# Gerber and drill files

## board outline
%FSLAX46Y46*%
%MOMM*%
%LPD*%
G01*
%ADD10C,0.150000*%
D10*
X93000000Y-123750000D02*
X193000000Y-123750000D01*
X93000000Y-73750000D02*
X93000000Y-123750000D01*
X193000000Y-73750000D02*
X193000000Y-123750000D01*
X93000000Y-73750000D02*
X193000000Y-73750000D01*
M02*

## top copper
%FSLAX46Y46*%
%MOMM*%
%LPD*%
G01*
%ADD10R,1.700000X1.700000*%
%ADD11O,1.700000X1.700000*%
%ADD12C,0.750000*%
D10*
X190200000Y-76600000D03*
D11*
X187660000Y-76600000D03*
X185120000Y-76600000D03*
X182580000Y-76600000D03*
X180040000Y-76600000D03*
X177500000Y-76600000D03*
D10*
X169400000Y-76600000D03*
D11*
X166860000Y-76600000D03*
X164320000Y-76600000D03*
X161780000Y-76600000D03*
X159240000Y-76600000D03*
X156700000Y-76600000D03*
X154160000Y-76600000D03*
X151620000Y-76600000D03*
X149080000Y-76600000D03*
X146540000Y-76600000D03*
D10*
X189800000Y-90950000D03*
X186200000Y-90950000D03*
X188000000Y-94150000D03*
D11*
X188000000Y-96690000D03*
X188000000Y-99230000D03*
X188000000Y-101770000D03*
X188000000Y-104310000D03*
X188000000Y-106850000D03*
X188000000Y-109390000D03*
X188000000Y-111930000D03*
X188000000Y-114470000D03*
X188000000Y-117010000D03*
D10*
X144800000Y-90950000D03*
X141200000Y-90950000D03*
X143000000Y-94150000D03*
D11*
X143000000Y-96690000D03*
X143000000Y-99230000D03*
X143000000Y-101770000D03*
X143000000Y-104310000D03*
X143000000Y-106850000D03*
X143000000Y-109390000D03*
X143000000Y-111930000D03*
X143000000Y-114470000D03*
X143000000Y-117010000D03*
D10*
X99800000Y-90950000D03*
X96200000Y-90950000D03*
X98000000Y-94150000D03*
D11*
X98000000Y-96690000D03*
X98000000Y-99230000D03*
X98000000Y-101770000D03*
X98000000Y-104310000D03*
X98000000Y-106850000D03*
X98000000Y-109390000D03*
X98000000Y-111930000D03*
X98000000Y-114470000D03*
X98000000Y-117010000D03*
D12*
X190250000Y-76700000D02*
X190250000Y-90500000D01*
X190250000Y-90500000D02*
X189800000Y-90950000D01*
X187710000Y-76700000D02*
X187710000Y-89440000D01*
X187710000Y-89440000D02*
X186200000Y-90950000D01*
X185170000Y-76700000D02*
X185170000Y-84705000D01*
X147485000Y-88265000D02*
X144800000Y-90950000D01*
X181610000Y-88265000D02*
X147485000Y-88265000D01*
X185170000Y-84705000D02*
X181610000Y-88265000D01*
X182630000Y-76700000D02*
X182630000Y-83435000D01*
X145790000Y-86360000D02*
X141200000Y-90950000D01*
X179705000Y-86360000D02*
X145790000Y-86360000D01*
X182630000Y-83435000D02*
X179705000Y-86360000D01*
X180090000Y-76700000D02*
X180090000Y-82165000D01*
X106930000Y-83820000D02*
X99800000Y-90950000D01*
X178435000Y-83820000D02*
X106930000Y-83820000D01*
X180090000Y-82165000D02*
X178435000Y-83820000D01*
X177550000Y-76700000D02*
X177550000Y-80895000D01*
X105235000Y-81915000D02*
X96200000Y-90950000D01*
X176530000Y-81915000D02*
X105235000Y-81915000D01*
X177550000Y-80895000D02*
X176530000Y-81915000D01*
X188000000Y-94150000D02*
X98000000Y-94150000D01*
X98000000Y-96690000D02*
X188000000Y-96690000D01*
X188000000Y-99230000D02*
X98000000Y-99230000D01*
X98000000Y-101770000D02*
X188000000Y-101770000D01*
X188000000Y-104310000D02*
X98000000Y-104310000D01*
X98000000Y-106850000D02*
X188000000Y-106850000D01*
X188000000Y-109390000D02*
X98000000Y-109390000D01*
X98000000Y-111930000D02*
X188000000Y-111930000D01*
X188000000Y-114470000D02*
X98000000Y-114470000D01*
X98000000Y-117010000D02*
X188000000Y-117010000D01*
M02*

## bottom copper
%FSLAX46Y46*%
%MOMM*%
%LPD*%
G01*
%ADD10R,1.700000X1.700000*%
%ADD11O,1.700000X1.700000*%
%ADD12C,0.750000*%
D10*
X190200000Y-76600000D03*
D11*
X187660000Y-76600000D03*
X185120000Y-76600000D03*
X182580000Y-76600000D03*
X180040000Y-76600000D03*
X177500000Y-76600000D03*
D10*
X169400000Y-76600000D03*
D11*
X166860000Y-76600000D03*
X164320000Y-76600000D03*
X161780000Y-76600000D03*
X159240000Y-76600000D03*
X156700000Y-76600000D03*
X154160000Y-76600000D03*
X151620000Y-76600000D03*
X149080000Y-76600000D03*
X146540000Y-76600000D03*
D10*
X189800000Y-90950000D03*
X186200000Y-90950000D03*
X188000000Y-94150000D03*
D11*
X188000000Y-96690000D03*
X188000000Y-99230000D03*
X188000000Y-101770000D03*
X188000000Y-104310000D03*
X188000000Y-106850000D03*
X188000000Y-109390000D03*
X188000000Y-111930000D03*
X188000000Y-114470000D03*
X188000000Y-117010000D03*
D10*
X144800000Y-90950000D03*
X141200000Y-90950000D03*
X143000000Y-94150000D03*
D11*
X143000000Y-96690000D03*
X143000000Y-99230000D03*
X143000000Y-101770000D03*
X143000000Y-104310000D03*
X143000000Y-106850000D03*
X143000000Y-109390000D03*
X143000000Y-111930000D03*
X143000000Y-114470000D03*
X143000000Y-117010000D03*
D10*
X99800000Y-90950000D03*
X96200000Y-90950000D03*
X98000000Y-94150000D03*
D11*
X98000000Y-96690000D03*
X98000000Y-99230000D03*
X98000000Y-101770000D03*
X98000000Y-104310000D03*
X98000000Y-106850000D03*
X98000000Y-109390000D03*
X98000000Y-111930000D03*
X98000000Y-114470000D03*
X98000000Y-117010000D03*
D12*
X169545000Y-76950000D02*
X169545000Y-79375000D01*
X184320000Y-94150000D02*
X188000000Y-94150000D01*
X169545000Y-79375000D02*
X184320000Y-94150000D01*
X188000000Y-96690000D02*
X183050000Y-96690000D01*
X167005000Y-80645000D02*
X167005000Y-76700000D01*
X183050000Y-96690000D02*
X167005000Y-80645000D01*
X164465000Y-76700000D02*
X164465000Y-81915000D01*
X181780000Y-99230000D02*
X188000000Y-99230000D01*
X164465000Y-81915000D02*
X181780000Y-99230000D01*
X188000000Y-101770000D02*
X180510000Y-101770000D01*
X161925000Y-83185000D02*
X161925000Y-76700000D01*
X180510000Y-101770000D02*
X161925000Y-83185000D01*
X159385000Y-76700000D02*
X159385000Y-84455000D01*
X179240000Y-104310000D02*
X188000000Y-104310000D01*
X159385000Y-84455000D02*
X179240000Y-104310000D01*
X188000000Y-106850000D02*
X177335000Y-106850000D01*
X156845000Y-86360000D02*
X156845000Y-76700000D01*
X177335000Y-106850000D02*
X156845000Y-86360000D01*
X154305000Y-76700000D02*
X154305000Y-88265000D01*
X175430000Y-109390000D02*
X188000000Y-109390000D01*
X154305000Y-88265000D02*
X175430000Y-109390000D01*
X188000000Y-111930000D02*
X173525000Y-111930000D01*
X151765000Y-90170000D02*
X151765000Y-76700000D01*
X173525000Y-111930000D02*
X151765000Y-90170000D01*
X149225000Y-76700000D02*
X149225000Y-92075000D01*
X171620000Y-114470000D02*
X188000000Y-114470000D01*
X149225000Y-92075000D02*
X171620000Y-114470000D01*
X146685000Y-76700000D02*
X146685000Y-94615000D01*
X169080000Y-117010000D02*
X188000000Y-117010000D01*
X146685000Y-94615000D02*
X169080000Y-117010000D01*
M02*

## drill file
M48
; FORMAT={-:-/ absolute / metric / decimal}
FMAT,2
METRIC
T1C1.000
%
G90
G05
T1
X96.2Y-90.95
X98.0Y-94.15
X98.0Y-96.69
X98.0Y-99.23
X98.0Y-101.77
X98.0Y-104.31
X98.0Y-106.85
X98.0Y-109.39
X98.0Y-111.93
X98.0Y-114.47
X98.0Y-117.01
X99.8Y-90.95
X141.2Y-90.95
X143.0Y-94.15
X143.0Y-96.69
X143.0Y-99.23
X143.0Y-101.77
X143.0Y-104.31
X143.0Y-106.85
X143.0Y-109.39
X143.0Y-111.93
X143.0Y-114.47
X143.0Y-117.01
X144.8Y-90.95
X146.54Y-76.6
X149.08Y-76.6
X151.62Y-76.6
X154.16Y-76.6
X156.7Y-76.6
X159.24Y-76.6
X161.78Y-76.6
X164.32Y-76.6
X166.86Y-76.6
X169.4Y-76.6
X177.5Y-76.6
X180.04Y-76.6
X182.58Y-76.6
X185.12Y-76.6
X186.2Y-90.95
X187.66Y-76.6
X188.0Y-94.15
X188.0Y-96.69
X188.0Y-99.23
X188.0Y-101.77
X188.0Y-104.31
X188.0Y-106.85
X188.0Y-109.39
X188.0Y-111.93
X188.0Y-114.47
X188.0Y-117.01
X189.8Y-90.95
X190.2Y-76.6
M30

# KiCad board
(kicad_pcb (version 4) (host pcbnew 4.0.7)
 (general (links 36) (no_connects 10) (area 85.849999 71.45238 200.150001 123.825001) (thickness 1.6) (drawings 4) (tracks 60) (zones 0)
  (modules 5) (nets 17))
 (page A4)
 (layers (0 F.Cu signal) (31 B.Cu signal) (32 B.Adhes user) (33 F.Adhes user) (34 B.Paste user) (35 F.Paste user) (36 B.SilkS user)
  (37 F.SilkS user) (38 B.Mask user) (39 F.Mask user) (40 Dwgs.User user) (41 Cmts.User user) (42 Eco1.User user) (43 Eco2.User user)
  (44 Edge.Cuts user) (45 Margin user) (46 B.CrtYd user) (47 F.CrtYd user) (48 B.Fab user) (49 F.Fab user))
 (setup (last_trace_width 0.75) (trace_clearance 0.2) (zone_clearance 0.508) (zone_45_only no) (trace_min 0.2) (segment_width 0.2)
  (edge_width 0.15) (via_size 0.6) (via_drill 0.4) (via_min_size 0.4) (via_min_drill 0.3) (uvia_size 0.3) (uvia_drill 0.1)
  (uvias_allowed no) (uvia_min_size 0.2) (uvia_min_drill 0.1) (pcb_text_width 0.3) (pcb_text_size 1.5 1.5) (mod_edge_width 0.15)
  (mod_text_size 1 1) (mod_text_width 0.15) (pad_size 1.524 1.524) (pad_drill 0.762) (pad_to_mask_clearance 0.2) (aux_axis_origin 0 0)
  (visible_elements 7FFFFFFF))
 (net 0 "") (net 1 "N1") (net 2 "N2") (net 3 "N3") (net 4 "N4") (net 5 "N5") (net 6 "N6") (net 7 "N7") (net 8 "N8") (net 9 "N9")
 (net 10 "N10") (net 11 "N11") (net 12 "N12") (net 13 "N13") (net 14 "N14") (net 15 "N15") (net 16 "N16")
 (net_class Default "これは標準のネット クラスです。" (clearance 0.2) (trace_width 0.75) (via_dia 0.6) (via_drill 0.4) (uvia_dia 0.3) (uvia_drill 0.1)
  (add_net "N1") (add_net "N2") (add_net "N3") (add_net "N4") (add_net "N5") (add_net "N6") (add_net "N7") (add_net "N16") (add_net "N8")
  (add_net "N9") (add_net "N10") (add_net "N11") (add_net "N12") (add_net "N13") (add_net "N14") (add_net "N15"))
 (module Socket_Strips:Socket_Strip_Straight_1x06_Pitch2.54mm (layer F.Cu) (at 190.2 76.6 270)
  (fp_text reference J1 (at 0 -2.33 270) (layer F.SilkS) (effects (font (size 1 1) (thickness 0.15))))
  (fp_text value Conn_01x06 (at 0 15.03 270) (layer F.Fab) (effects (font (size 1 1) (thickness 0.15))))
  (pad 1 thru_hole rect (at 0 0 270) (size 1.7 1.7) (drill 1) (layers *.Cu *.Mask) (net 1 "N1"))
  (pad 2 thru_hole oval (at 0 2.54 270) (size 1.7 1.7) (drill 1) (layers *.Cu *.Mask) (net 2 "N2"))
  (pad 3 thru_hole oval (at 0 5.08 270) (size 1.7 1.7) (drill 1) (layers *.Cu *.Mask) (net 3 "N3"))
  (pad 4 thru_hole oval (at 0 7.62 270) (size 1.7 1.7) (drill 1) (layers *.Cu *.Mask) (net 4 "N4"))
  (pad 5 thru_hole oval (at 0 10.16 270) (size 1.7 1.7) (drill 1) (layers *.Cu *.Mask) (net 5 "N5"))
  (pad 6 thru_hole oval (at 0 12.7 270) (size 1.7 1.7) (drill 1) (layers *.Cu *.Mask) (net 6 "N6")))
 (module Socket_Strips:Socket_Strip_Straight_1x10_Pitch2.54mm (layer F.Cu) (at 169.4 76.6 270)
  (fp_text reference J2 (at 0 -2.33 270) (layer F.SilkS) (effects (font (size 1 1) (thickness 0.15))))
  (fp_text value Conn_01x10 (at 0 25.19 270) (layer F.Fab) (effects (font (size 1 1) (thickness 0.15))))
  (pad 1 thru_hole rect (at 0 0 270) (size 1.7 1.7) (drill 1) (layers *.Cu *.Mask) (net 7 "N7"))
  (pad 2 thru_hole oval (at 0 2.54 270) (size 1.7 1.7) (drill 1) (layers *.Cu *.Mask) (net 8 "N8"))
  (pad 3 thru_hole oval (at 0 5.08 270) (size 1.7 1.7) (drill 1) (layers *.Cu *.Mask) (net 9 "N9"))
  (pad 4 thru_hole oval (at 0 7.62 270) (size 1.7 1.7) (drill 1) (layers *.Cu *.Mask) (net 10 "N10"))
  (pad 5 thru_hole oval (at 0 10.16 270) (size 1.7 1.7) (drill 1) (layers *.Cu *.Mask) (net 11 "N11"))
  (pad 6 thru_hole oval (at 0 12.7 270) (size 1.7 1.7) (drill 1) (layers *.Cu *.Mask) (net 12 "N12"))
  (pad 7 thru_hole oval (at 0 15.24 270) (size 1.7 1.7) (drill 1) (layers *.Cu *.Mask) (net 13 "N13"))
  (pad 8 thru_hole oval (at 0 17.78 270) (size 1.7 1.7) (drill 1) (layers *.Cu *.Mask) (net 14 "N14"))
  (pad 9 thru_hole oval (at 0 20.32 270) (size 1.7 1.7) (drill 1) (layers *.Cu *.Mask) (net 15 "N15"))
  (pad 10 thru_hole oval (at 0 22.86 270) (size 1.7 1.7) (drill 1) (layers *.Cu *.Mask) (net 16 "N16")))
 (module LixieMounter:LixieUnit (layer F.Cu) (at 188 94.55)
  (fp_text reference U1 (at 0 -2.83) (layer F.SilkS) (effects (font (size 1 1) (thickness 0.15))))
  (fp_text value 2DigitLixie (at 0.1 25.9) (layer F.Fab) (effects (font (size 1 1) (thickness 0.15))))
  (pad 1 thru_hole rect (at 1.8 -3.6) (size 1.7 1.7) (drill 1) (layers *.Cu *.Mask) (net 1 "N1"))
  (pad 2 thru_hole rect (at -1.8 -3.6) (size 1.7 1.7) (drill 1) (layers *.Cu *.Mask) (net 2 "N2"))
  (pad 3 thru_hole rect (at 0 -0.4) (size 1.7 1.7) (drill 1) (layers *.Cu *.Mask) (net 7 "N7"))
  (pad 4 thru_hole oval (at 0 2.14) (size 1.7 1.7) (drill 1) (layers *.Cu *.Mask) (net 8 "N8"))
  (pad 5 thru_hole oval (at 0 4.68) (size 1.7 1.7) (drill 1) (layers *.Cu *.Mask) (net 9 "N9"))
  (pad 6 thru_hole oval (at 0 7.22) (size 1.7 1.7) (drill 1) (layers *.Cu *.Mask) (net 10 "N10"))
  (pad 7 thru_hole oval (at 0 9.76) (size 1.7 1.7) (drill 1) (layers *.Cu *.Mask) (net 11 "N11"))
  (pad 8 thru_hole oval (at 0 12.3) (size 1.7 1.7) (drill 1) (layers *.Cu *.Mask) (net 12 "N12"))
  (pad 9 thru_hole oval (at 0 14.84) (size 1.7 1.7) (drill 1) (layers *.Cu *.Mask) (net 13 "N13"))
  (pad 10 thru_hole oval (at 0 17.38) (size 1.7 1.7) (drill 1) (layers *.Cu *.Mask) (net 14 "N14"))
  (pad 11 thru_hole oval (at 0 19.92) (size 1.7 1.7) (drill 1) (layers *.Cu *.Mask) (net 15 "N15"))
  (pad 12 thru_hole oval (at 0 22.46) (size 1.7 1.7) (drill 1) (layers *.Cu *.Mask) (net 16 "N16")))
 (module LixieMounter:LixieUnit (layer F.Cu) (at 143 94.55)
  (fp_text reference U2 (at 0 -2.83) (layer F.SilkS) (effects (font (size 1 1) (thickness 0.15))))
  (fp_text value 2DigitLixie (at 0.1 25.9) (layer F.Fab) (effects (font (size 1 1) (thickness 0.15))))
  (pad 1 thru_hole rect (at 1.8 -3.6) (size 1.7 1.7) (drill 1) (layers *.Cu *.Mask) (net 3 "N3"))
  (pad 2 thru_hole rect (at -1.8 -3.6) (size 1.7 1.7) (drill 1) (layers *.Cu *.Mask) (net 4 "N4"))
  (pad 3 thru_hole rect (at 0 -0.4) (size 1.7 1.7) (drill 1) (layers *.Cu *.Mask) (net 7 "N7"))
  (pad 4 thru_hole oval (at 0 2.14) (size 1.7 1.7) (drill 1) (layers *.Cu *.Mask) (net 8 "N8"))
  (pad 5 thru_hole oval (at 0 4.68) (size 1.7 1.7) (drill 1) (layers *.Cu *.Mask) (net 9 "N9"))
  (pad 6 thru_hole oval (at 0 7.22) (size 1.7 1.7) (drill 1) (layers *.Cu *.Mask) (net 10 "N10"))
  (pad 7 thru_hole oval (at 0 9.76) (size 1.7 1.7) (drill 1) (layers *.Cu *.Mask) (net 11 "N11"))
  (pad 8 thru_hole oval (at 0 12.3) (size 1.7 1.7) (drill 1) (layers *.Cu *.Mask) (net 12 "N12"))
  (pad 9 thru_hole oval (at 0 14.84) (size 1.7 1.7) (drill 1) (layers *.Cu *.Mask) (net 13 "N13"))
  (pad 10 thru_hole oval (at 0 17.38) (size 1.7 1.7) (drill 1) (layers *.Cu *.Mask) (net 14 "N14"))
  (pad 11 thru_hole oval (at 0 19.92) (size 1.7 1.7) (drill 1) (layers *.Cu *.Mask) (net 15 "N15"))
  (pad 12 thru_hole oval (at 0 22.46) (size 1.7 1.7) (drill 1) (layers *.Cu *.Mask) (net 16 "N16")))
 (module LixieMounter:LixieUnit (layer F.Cu) (at 98 94.55)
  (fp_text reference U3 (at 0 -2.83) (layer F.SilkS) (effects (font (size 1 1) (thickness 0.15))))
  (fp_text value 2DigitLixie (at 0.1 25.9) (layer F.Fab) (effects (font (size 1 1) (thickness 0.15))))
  (pad 1 thru_hole rect (at 1.8 -3.6) (size 1.7 1.7) (drill 1) (layers *.Cu *.Mask) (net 5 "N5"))
  (pad 2 thru_hole rect (at -1.8 -3.6) (size 1.7 1.7) (drill 1) (layers *.Cu *.Mask) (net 6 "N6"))
  (pad 3 thru_hole rect (at 0 -0.4) (size 1.7 1.7) (drill 1) (layers *.Cu *.Mask) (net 7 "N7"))
  (pad 4 thru_hole oval (at 0 2.14) (size 1.7 1.7) (drill 1) (layers *.Cu *.Mask) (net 8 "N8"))
  (pad 5 thru_hole oval (at 0 4.68) (size 1.7 1.7) (drill 1) (layers *.Cu *.Mask) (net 9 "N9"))
  (pad 6 thru_hole oval (at 0 7.22) (size 1.7 1.7) (drill 1) (layers *.Cu *.Mask) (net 10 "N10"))
  (pad 7 thru_hole oval (at 0 9.76) (size 1.7 1.7) (drill 1) (layers *.Cu *.Mask) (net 11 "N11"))
  (pad 8 thru_hole oval (at 0 12.3) (size 1.7 1.7) (drill 1) (layers *.Cu *.Mask) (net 12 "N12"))
  (pad 9 thru_hole oval (at 0 14.84) (size 1.7 1.7) (drill 1) (layers *.Cu *.Mask) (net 13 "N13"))
  (pad 10 thru_hole oval (at 0 17.38) (size 1.7 1.7) (drill 1) (layers *.Cu *.Mask) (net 14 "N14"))
  (pad 11 thru_hole oval (at 0 19.92) (size 1.7 1.7) (drill 1) (layers *.Cu *.Mask) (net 15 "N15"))
  (pad 12 thru_hole oval (at 0 22.46) (size 1.7 1.7) (drill 1) (layers *.Cu *.Mask) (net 16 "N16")))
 (gr_line (start 93 123.75) (end 193 123.75) (angle 90) (layer Edge.Cuts) (width 0.15))
 (gr_line (start 93 73.75) (end 93 123.75) (angle 90) (layer Edge.Cuts) (width 0.15))
 (gr_line (start 193 73.75) (end 193 123.75) (angle 90) (layer Edge.Cuts) (width 0.15))
 (gr_line (start 93 73.75) (end 193 73.75) (angle 90) (layer Edge.Cuts) (width 0.15))
 (segment (start 190.25 76.7) (end 190.25 90.5) (width 0.75) (layer F.Cu) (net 1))
 (segment (start 190.25 90.5) (end 189.8 90.95) (width 0.75) (layer F.Cu) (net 1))
 (segment (start 187.71 76.7) (end 187.71 89.44) (width 0.75) (layer F.Cu) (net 2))
 (segment (start 187.71 89.44) (end 186.2 90.95) (width 0.75) (layer F.Cu) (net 2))
 (segment (start 185.17 76.7) (end 185.17 84.705) (width 0.75) (layer F.Cu) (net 3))
 (segment (start 147.485 88.265) (end 144.8 90.95) (width 0.75) (layer F.Cu) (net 3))
 (segment (start 181.61 88.265) (end 147.485 88.265) (width 0.75) (layer F.Cu) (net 3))
 (segment (start 185.17 84.705) (end 181.61 88.265) (width 0.75) (layer F.Cu) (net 3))
 (segment (start 182.63 76.7) (end 182.63 83.435) (width 0.75) (layer F.Cu) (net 4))
 (segment (start 145.79 86.36) (end 141.2 90.95) (width 0.75) (layer F.Cu) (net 4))
 (segment (start 179.705 86.36) (end 145.79 86.36) (width 0.75) (layer F.Cu) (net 4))
 (segment (start 182.63 83.435) (end 179.705 86.36) (width 0.75) (layer F.Cu) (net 4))
 (segment (start 180.09 76.7) (end 180.09 82.165) (width 0.75) (layer F.Cu) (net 5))
 (segment (start 106.93 83.82) (end 99.8 90.95) (width 0.75) (layer F.Cu) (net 5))
 (segment (start 178.435 83.82) (end 106.93 83.82) (width 0.75) (layer F.Cu) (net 5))
 (segment (start 180.09 82.165) (end 178.435 83.82) (width 0.75) (layer F.Cu) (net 5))
 (segment (start 177.55 76.7) (end 177.55 80.895) (width 0.75) (layer F.Cu) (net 6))
 (segment (start 105.235 81.915) (end 96.2 90.95) (width 0.75) (layer F.Cu) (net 6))
 (segment (start 176.53 81.915) (end 105.235 81.915) (width 0.75) (layer F.Cu) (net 6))
 (segment (start 177.55 80.895) (end 176.53 81.915) (width 0.75) (layer F.Cu) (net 6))
 (segment (start 169.545 76.95) (end 169.545 79.375) (width 0.75) (layer B.Cu) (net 7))
 (segment (start 184.32 94.15) (end 188 94.15) (width 0.75) (layer B.Cu) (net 7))
 (segment (start 169.545 79.375) (end 184.32 94.15) (width 0.75) (layer B.Cu) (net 7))
 (segment (start 188 94.15) (end 98 94.15) (width 0.75) (layer F.Cu) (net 7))
 (segment (start 188 96.69) (end 183.05 96.69) (width 0.75) (layer B.Cu) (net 8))
 (segment (start 167.005 80.645) (end 167.005 76.7) (width 0.75) (layer B.Cu) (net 8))
 (segment (start 183.05 96.69) (end 167.005 80.645) (width 0.75) (layer B.Cu) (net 8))
 (segment (start 98 96.69) (end 188 96.69) (width 0.75) (layer F.Cu) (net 8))
 (segment (start 164.465 76.7) (end 164.465 81.915) (width 0.75) (layer B.Cu) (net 9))
 (segment (start 181.78 99.23) (end 188 99.23) (width 0.75) (layer B.Cu) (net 9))
 (segment (start 164.465 81.915) (end 181.78 99.23) (width 0.75) (layer B.Cu) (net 9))
 (segment (start 188 99.23) (end 98 99.23) (width 0.75) (layer F.Cu) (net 9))
 (segment (start 188 101.77) (end 180.51 101.77) (width 0.75) (layer B.Cu) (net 10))
 (segment (start 161.925 83.185) (end 161.925 76.7) (width 0.75) (layer B.Cu) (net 10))
 (segment (start 180.51 101.77) (end 161.925 83.185) (width 0.75) (layer B.Cu) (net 10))
 (segment (start 98 101.77) (end 188 101.77) (width 0.75) (layer F.Cu) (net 10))
 (segment (start 159.385 76.7) (end 159.385 84.455) (width 0.75) (layer B.Cu) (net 11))
 (segment (start 179.24 104.31) (end 188 104.31) (width 0.75) (layer B.Cu) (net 11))
 (segment (start 159.385 84.455) (end 179.24 104.31) (width 0.75) (layer B.Cu) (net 11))
 (segment (start 188 104.31) (end 98 104.31) (width 0.75) (layer F.Cu) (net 11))
 (segment (start 188 106.85) (end 177.335 106.85) (width 0.75) (layer B.Cu) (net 12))
 (segment (start 156.845 86.36) (end 156.845 76.7) (width 0.75) (layer B.Cu) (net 12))
 (segment (start 177.335 106.85) (end 156.845 86.36) (width 0.75) (layer B.Cu) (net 12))
 (segment (start 98 106.85) (end 188 106.85) (width 0.75) (layer F.Cu) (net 12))
 (segment (start 154.305 76.7) (end 154.305 88.265) (width 0.75) (layer B.Cu) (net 13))
 (segment (start 175.43 109.39) (end 188 109.39) (width 0.75) (layer B.Cu) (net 13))
 (segment (start 154.305 88.265) (end 175.43 109.39) (width 0.75) (layer B.Cu) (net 13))
 (segment (start 188 109.39) (end 98 109.39) (width 0.75) (layer F.Cu) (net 13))
 (segment (start 188 111.93) (end 173.525 111.93) (width 0.75) (layer B.Cu) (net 14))
 (segment (start 151.765 90.17) (end 151.765 76.7) (width 0.75) (layer B.Cu) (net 14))
 (segment (start 173.525 111.93) (end 151.765 90.17) (width 0.75) (layer B.Cu) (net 14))
 (segment (start 98 111.93) (end 188 111.93) (width 0.75) (layer F.Cu) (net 14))
 (segment (start 149.225 76.7) (end 149.225 92.075) (width 0.75) (layer B.Cu) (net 15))
 (segment (start 171.62 114.47) (end 188 114.47) (width 0.75) (layer B.Cu) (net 15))
 (segment (start 149.225 92.075) (end 171.62 114.47) (width 0.75) (layer B.Cu) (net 15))
 (segment (start 188 114.47) (end 98 114.47) (width 0.75) (layer F.Cu) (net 15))
 (segment (start 146.685 76.7) (end 146.685 94.615) (width 0.75) (layer B.Cu) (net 16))
 (segment (start 169.08 117.01) (end 188 117.01) (width 0.75) (layer B.Cu) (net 16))
 (segment (start 146.685 94.615) (end 169.08 117.01) (width 0.75) (layer B.Cu) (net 16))
 (segment (start 98 117.01) (end 188 117.01) (width 0.75) (layer F.Cu) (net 16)))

